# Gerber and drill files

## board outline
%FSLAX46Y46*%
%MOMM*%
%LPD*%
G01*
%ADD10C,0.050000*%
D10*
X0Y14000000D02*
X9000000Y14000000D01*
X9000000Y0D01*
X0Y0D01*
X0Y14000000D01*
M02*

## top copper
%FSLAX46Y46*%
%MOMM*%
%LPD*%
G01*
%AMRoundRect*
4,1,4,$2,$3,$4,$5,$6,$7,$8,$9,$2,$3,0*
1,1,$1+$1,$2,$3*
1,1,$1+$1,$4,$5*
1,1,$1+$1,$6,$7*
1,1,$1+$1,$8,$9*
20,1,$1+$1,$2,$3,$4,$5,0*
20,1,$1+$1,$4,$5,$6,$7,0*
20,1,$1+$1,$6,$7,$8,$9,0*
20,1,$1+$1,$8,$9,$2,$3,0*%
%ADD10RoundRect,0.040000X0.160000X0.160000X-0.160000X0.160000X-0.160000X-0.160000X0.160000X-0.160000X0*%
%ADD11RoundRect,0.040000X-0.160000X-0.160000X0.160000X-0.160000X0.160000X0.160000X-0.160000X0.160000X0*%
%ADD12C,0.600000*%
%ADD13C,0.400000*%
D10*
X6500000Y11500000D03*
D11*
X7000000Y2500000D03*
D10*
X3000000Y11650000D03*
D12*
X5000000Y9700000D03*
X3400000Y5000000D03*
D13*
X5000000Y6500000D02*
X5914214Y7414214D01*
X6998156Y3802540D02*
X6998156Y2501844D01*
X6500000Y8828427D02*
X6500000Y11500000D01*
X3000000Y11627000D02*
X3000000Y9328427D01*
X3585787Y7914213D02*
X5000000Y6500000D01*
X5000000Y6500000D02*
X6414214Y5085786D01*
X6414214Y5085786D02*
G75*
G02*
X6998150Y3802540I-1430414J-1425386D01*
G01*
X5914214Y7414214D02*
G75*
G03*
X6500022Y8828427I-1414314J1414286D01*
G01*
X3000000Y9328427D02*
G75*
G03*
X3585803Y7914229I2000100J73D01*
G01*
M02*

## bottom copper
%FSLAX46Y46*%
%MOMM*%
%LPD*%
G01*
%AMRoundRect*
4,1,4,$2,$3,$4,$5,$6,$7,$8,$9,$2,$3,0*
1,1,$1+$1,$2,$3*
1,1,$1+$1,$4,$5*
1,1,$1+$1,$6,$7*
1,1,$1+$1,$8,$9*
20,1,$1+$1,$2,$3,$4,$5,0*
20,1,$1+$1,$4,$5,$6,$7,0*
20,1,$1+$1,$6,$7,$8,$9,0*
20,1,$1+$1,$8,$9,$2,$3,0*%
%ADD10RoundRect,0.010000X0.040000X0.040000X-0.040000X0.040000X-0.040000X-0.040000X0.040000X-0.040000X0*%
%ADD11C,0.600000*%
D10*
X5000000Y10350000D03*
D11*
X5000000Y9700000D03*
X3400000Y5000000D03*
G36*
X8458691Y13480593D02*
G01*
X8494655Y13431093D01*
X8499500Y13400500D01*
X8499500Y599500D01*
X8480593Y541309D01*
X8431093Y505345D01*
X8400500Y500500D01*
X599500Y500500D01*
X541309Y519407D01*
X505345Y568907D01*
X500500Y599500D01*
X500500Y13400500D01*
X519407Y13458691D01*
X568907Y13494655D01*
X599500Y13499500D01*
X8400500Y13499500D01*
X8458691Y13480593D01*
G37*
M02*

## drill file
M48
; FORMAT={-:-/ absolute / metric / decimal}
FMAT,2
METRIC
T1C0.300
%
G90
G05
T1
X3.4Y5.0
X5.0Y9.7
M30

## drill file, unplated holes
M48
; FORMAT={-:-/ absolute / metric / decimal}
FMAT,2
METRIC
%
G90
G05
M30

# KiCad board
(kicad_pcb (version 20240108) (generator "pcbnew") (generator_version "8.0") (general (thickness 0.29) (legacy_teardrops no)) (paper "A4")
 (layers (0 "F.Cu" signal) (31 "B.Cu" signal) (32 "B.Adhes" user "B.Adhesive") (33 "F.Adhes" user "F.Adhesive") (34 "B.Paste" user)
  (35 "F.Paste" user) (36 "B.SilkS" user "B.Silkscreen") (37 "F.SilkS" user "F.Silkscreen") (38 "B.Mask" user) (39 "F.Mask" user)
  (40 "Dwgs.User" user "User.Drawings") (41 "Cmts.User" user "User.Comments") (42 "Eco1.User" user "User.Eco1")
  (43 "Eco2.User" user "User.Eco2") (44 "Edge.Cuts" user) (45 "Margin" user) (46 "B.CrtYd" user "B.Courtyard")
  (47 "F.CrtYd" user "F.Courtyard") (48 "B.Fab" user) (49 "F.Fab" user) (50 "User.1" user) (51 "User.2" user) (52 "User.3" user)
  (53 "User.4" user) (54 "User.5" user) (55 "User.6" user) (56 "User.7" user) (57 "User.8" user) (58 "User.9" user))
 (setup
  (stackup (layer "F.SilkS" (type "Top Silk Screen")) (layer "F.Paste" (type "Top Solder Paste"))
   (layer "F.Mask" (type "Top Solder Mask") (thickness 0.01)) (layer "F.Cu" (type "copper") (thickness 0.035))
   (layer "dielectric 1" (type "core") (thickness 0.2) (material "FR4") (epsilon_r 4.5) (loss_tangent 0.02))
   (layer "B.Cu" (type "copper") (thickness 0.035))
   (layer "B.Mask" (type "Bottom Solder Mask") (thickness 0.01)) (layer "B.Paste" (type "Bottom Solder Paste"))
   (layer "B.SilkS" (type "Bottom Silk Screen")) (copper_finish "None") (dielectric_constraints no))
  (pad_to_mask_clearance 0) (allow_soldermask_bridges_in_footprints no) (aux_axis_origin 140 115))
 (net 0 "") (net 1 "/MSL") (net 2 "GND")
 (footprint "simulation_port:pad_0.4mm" (layer "F.Cu") (at 147 112.5)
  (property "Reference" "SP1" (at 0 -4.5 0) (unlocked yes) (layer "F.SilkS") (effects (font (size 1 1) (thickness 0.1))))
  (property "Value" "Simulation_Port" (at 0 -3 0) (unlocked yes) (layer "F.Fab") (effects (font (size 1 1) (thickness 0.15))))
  (pad "1" smd roundrect (at 0 0) (size 0.4 0.4) (layers "F.Cu" "F.Paste" "F.Mask") (roundrect_rratio 0.1) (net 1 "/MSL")
   (thermal_bridge_angle 45)
   (teardrops (best_length_ratio 0.5) (max_length 1) (best_width_ratio 1) (max_width 2) (curve_points 0) (filter_ratio 0.9) (enabled yes)
    (allow_two_segments yes) (prefer_zone_connections yes))))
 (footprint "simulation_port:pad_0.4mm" (layer "F.Cu") (at 146.5 103.5 180)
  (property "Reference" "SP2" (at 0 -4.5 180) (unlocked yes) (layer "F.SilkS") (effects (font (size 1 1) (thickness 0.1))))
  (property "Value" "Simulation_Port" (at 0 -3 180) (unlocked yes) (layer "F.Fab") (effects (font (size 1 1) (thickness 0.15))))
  (pad "1" smd roundrect (at 0 0 180) (size 0.4 0.4) (layers "F.Cu" "F.Paste" "F.Mask") (roundrect_rratio 0.1) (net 1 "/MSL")
   (thermal_bridge_angle 45)
   (teardrops (best_length_ratio 0.5) (max_length 1) (best_width_ratio 1) (max_width 2) (curve_points 0) (filter_ratio 0.9) (enabled yes)
    (allow_two_segments yes) (prefer_zone_connections yes))))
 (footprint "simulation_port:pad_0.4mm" (layer "F.Cu") (at 143 103.35 180)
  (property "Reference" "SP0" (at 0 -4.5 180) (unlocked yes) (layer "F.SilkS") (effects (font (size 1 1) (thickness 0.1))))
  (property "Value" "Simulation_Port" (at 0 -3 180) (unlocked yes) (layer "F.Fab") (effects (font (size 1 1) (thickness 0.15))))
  (pad "1" smd roundrect (at 0 0 180) (size 0.4 0.4) (layers "F.Cu" "F.Paste" "F.Mask") (roundrect_rratio 0.1) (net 1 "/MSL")
   (thermal_bridge_angle 45)
   (teardrops (best_length_ratio 0.5) (max_length 1) (best_width_ratio 1) (max_width 2) (curve_points 0) (filter_ratio 0.9) (enabled yes)
    (allow_two_segments yes) (prefer_zone_connections yes))))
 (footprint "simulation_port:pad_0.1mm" (layer "B.Cu") (at 145 104.65 180)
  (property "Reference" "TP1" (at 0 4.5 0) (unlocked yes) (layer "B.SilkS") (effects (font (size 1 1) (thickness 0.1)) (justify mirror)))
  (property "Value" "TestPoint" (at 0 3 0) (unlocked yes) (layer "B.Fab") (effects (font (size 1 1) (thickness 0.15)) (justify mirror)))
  (pad "1" smd roundrect (at 0 0 180) (size 0.1 0.1) (layers "B.Cu" "B.Paste" "B.Mask") (roundrect_rratio 0.1) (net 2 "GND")
   (thermal_bridge_angle 45)
   (teardrops (best_length_ratio 0.5) (max_length 1) (best_width_ratio 1) (max_width 2) (curve_points 0) (filter_ratio 0.9) (enabled yes)
    (allow_two_segments yes) (prefer_zone_connections yes))))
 (gr_rect (start 140 101) (end 149 115) (stroke (width 0.05) (type solid)) (fill none) (layer "Edge.Cuts"))
 (segment (start 145 108.5) (end 145.914214 107.585786) (width 0.4) (layer "F.Cu") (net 1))
 (segment (start 146.998156 111.19746) (end 146.998156 112.498156) (width 0.4) (layer "F.Cu") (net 1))
 (segment (start 146.5 106.171573) (end 146.5 103.5) (width 0.4) (layer "F.Cu") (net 1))
 (segment (start 143 103.373) (end 143 105.671573) (width 0.4) (layer "F.Cu") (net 1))
 (segment (start 143.585787 107.085787) (end 145 108.5) (width 0.4) (layer "F.Cu") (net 1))
 (segment (start 145 108.5) (end 146.414214 109.914214) (width 0.4) (layer "F.Cu") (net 1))
 (arc (start 146.414214 109.914214) (mid 146.82172 110.503015) (end 146.998156 111.19746) (width 0.4) (layer "F.Cu") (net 1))
 (arc (start 145.914214 107.585786) (mid 146.34775 106.936938) (end 146.5 106.171573) (width 0.4) (layer "F.Cu") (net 1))
 (arc (start 143 105.671573) (mid 143.15225 106.436939) (end 143.585787 107.085787) (width 0.4) (layer "F.Cu") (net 1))
 (via (at 145 105.3) (size 0.6) (drill 0.3) (layers "F.Cu" "B.Cu") (free yes) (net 2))
 (via (at 143.4 110) (size 0.6) (drill 0.3) (layers "F.Cu" "B.Cu") (free yes) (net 2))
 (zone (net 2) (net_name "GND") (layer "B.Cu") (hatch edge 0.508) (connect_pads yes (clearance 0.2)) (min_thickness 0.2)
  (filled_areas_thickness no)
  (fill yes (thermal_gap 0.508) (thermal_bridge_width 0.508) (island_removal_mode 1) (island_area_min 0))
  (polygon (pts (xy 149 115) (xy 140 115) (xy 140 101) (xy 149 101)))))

